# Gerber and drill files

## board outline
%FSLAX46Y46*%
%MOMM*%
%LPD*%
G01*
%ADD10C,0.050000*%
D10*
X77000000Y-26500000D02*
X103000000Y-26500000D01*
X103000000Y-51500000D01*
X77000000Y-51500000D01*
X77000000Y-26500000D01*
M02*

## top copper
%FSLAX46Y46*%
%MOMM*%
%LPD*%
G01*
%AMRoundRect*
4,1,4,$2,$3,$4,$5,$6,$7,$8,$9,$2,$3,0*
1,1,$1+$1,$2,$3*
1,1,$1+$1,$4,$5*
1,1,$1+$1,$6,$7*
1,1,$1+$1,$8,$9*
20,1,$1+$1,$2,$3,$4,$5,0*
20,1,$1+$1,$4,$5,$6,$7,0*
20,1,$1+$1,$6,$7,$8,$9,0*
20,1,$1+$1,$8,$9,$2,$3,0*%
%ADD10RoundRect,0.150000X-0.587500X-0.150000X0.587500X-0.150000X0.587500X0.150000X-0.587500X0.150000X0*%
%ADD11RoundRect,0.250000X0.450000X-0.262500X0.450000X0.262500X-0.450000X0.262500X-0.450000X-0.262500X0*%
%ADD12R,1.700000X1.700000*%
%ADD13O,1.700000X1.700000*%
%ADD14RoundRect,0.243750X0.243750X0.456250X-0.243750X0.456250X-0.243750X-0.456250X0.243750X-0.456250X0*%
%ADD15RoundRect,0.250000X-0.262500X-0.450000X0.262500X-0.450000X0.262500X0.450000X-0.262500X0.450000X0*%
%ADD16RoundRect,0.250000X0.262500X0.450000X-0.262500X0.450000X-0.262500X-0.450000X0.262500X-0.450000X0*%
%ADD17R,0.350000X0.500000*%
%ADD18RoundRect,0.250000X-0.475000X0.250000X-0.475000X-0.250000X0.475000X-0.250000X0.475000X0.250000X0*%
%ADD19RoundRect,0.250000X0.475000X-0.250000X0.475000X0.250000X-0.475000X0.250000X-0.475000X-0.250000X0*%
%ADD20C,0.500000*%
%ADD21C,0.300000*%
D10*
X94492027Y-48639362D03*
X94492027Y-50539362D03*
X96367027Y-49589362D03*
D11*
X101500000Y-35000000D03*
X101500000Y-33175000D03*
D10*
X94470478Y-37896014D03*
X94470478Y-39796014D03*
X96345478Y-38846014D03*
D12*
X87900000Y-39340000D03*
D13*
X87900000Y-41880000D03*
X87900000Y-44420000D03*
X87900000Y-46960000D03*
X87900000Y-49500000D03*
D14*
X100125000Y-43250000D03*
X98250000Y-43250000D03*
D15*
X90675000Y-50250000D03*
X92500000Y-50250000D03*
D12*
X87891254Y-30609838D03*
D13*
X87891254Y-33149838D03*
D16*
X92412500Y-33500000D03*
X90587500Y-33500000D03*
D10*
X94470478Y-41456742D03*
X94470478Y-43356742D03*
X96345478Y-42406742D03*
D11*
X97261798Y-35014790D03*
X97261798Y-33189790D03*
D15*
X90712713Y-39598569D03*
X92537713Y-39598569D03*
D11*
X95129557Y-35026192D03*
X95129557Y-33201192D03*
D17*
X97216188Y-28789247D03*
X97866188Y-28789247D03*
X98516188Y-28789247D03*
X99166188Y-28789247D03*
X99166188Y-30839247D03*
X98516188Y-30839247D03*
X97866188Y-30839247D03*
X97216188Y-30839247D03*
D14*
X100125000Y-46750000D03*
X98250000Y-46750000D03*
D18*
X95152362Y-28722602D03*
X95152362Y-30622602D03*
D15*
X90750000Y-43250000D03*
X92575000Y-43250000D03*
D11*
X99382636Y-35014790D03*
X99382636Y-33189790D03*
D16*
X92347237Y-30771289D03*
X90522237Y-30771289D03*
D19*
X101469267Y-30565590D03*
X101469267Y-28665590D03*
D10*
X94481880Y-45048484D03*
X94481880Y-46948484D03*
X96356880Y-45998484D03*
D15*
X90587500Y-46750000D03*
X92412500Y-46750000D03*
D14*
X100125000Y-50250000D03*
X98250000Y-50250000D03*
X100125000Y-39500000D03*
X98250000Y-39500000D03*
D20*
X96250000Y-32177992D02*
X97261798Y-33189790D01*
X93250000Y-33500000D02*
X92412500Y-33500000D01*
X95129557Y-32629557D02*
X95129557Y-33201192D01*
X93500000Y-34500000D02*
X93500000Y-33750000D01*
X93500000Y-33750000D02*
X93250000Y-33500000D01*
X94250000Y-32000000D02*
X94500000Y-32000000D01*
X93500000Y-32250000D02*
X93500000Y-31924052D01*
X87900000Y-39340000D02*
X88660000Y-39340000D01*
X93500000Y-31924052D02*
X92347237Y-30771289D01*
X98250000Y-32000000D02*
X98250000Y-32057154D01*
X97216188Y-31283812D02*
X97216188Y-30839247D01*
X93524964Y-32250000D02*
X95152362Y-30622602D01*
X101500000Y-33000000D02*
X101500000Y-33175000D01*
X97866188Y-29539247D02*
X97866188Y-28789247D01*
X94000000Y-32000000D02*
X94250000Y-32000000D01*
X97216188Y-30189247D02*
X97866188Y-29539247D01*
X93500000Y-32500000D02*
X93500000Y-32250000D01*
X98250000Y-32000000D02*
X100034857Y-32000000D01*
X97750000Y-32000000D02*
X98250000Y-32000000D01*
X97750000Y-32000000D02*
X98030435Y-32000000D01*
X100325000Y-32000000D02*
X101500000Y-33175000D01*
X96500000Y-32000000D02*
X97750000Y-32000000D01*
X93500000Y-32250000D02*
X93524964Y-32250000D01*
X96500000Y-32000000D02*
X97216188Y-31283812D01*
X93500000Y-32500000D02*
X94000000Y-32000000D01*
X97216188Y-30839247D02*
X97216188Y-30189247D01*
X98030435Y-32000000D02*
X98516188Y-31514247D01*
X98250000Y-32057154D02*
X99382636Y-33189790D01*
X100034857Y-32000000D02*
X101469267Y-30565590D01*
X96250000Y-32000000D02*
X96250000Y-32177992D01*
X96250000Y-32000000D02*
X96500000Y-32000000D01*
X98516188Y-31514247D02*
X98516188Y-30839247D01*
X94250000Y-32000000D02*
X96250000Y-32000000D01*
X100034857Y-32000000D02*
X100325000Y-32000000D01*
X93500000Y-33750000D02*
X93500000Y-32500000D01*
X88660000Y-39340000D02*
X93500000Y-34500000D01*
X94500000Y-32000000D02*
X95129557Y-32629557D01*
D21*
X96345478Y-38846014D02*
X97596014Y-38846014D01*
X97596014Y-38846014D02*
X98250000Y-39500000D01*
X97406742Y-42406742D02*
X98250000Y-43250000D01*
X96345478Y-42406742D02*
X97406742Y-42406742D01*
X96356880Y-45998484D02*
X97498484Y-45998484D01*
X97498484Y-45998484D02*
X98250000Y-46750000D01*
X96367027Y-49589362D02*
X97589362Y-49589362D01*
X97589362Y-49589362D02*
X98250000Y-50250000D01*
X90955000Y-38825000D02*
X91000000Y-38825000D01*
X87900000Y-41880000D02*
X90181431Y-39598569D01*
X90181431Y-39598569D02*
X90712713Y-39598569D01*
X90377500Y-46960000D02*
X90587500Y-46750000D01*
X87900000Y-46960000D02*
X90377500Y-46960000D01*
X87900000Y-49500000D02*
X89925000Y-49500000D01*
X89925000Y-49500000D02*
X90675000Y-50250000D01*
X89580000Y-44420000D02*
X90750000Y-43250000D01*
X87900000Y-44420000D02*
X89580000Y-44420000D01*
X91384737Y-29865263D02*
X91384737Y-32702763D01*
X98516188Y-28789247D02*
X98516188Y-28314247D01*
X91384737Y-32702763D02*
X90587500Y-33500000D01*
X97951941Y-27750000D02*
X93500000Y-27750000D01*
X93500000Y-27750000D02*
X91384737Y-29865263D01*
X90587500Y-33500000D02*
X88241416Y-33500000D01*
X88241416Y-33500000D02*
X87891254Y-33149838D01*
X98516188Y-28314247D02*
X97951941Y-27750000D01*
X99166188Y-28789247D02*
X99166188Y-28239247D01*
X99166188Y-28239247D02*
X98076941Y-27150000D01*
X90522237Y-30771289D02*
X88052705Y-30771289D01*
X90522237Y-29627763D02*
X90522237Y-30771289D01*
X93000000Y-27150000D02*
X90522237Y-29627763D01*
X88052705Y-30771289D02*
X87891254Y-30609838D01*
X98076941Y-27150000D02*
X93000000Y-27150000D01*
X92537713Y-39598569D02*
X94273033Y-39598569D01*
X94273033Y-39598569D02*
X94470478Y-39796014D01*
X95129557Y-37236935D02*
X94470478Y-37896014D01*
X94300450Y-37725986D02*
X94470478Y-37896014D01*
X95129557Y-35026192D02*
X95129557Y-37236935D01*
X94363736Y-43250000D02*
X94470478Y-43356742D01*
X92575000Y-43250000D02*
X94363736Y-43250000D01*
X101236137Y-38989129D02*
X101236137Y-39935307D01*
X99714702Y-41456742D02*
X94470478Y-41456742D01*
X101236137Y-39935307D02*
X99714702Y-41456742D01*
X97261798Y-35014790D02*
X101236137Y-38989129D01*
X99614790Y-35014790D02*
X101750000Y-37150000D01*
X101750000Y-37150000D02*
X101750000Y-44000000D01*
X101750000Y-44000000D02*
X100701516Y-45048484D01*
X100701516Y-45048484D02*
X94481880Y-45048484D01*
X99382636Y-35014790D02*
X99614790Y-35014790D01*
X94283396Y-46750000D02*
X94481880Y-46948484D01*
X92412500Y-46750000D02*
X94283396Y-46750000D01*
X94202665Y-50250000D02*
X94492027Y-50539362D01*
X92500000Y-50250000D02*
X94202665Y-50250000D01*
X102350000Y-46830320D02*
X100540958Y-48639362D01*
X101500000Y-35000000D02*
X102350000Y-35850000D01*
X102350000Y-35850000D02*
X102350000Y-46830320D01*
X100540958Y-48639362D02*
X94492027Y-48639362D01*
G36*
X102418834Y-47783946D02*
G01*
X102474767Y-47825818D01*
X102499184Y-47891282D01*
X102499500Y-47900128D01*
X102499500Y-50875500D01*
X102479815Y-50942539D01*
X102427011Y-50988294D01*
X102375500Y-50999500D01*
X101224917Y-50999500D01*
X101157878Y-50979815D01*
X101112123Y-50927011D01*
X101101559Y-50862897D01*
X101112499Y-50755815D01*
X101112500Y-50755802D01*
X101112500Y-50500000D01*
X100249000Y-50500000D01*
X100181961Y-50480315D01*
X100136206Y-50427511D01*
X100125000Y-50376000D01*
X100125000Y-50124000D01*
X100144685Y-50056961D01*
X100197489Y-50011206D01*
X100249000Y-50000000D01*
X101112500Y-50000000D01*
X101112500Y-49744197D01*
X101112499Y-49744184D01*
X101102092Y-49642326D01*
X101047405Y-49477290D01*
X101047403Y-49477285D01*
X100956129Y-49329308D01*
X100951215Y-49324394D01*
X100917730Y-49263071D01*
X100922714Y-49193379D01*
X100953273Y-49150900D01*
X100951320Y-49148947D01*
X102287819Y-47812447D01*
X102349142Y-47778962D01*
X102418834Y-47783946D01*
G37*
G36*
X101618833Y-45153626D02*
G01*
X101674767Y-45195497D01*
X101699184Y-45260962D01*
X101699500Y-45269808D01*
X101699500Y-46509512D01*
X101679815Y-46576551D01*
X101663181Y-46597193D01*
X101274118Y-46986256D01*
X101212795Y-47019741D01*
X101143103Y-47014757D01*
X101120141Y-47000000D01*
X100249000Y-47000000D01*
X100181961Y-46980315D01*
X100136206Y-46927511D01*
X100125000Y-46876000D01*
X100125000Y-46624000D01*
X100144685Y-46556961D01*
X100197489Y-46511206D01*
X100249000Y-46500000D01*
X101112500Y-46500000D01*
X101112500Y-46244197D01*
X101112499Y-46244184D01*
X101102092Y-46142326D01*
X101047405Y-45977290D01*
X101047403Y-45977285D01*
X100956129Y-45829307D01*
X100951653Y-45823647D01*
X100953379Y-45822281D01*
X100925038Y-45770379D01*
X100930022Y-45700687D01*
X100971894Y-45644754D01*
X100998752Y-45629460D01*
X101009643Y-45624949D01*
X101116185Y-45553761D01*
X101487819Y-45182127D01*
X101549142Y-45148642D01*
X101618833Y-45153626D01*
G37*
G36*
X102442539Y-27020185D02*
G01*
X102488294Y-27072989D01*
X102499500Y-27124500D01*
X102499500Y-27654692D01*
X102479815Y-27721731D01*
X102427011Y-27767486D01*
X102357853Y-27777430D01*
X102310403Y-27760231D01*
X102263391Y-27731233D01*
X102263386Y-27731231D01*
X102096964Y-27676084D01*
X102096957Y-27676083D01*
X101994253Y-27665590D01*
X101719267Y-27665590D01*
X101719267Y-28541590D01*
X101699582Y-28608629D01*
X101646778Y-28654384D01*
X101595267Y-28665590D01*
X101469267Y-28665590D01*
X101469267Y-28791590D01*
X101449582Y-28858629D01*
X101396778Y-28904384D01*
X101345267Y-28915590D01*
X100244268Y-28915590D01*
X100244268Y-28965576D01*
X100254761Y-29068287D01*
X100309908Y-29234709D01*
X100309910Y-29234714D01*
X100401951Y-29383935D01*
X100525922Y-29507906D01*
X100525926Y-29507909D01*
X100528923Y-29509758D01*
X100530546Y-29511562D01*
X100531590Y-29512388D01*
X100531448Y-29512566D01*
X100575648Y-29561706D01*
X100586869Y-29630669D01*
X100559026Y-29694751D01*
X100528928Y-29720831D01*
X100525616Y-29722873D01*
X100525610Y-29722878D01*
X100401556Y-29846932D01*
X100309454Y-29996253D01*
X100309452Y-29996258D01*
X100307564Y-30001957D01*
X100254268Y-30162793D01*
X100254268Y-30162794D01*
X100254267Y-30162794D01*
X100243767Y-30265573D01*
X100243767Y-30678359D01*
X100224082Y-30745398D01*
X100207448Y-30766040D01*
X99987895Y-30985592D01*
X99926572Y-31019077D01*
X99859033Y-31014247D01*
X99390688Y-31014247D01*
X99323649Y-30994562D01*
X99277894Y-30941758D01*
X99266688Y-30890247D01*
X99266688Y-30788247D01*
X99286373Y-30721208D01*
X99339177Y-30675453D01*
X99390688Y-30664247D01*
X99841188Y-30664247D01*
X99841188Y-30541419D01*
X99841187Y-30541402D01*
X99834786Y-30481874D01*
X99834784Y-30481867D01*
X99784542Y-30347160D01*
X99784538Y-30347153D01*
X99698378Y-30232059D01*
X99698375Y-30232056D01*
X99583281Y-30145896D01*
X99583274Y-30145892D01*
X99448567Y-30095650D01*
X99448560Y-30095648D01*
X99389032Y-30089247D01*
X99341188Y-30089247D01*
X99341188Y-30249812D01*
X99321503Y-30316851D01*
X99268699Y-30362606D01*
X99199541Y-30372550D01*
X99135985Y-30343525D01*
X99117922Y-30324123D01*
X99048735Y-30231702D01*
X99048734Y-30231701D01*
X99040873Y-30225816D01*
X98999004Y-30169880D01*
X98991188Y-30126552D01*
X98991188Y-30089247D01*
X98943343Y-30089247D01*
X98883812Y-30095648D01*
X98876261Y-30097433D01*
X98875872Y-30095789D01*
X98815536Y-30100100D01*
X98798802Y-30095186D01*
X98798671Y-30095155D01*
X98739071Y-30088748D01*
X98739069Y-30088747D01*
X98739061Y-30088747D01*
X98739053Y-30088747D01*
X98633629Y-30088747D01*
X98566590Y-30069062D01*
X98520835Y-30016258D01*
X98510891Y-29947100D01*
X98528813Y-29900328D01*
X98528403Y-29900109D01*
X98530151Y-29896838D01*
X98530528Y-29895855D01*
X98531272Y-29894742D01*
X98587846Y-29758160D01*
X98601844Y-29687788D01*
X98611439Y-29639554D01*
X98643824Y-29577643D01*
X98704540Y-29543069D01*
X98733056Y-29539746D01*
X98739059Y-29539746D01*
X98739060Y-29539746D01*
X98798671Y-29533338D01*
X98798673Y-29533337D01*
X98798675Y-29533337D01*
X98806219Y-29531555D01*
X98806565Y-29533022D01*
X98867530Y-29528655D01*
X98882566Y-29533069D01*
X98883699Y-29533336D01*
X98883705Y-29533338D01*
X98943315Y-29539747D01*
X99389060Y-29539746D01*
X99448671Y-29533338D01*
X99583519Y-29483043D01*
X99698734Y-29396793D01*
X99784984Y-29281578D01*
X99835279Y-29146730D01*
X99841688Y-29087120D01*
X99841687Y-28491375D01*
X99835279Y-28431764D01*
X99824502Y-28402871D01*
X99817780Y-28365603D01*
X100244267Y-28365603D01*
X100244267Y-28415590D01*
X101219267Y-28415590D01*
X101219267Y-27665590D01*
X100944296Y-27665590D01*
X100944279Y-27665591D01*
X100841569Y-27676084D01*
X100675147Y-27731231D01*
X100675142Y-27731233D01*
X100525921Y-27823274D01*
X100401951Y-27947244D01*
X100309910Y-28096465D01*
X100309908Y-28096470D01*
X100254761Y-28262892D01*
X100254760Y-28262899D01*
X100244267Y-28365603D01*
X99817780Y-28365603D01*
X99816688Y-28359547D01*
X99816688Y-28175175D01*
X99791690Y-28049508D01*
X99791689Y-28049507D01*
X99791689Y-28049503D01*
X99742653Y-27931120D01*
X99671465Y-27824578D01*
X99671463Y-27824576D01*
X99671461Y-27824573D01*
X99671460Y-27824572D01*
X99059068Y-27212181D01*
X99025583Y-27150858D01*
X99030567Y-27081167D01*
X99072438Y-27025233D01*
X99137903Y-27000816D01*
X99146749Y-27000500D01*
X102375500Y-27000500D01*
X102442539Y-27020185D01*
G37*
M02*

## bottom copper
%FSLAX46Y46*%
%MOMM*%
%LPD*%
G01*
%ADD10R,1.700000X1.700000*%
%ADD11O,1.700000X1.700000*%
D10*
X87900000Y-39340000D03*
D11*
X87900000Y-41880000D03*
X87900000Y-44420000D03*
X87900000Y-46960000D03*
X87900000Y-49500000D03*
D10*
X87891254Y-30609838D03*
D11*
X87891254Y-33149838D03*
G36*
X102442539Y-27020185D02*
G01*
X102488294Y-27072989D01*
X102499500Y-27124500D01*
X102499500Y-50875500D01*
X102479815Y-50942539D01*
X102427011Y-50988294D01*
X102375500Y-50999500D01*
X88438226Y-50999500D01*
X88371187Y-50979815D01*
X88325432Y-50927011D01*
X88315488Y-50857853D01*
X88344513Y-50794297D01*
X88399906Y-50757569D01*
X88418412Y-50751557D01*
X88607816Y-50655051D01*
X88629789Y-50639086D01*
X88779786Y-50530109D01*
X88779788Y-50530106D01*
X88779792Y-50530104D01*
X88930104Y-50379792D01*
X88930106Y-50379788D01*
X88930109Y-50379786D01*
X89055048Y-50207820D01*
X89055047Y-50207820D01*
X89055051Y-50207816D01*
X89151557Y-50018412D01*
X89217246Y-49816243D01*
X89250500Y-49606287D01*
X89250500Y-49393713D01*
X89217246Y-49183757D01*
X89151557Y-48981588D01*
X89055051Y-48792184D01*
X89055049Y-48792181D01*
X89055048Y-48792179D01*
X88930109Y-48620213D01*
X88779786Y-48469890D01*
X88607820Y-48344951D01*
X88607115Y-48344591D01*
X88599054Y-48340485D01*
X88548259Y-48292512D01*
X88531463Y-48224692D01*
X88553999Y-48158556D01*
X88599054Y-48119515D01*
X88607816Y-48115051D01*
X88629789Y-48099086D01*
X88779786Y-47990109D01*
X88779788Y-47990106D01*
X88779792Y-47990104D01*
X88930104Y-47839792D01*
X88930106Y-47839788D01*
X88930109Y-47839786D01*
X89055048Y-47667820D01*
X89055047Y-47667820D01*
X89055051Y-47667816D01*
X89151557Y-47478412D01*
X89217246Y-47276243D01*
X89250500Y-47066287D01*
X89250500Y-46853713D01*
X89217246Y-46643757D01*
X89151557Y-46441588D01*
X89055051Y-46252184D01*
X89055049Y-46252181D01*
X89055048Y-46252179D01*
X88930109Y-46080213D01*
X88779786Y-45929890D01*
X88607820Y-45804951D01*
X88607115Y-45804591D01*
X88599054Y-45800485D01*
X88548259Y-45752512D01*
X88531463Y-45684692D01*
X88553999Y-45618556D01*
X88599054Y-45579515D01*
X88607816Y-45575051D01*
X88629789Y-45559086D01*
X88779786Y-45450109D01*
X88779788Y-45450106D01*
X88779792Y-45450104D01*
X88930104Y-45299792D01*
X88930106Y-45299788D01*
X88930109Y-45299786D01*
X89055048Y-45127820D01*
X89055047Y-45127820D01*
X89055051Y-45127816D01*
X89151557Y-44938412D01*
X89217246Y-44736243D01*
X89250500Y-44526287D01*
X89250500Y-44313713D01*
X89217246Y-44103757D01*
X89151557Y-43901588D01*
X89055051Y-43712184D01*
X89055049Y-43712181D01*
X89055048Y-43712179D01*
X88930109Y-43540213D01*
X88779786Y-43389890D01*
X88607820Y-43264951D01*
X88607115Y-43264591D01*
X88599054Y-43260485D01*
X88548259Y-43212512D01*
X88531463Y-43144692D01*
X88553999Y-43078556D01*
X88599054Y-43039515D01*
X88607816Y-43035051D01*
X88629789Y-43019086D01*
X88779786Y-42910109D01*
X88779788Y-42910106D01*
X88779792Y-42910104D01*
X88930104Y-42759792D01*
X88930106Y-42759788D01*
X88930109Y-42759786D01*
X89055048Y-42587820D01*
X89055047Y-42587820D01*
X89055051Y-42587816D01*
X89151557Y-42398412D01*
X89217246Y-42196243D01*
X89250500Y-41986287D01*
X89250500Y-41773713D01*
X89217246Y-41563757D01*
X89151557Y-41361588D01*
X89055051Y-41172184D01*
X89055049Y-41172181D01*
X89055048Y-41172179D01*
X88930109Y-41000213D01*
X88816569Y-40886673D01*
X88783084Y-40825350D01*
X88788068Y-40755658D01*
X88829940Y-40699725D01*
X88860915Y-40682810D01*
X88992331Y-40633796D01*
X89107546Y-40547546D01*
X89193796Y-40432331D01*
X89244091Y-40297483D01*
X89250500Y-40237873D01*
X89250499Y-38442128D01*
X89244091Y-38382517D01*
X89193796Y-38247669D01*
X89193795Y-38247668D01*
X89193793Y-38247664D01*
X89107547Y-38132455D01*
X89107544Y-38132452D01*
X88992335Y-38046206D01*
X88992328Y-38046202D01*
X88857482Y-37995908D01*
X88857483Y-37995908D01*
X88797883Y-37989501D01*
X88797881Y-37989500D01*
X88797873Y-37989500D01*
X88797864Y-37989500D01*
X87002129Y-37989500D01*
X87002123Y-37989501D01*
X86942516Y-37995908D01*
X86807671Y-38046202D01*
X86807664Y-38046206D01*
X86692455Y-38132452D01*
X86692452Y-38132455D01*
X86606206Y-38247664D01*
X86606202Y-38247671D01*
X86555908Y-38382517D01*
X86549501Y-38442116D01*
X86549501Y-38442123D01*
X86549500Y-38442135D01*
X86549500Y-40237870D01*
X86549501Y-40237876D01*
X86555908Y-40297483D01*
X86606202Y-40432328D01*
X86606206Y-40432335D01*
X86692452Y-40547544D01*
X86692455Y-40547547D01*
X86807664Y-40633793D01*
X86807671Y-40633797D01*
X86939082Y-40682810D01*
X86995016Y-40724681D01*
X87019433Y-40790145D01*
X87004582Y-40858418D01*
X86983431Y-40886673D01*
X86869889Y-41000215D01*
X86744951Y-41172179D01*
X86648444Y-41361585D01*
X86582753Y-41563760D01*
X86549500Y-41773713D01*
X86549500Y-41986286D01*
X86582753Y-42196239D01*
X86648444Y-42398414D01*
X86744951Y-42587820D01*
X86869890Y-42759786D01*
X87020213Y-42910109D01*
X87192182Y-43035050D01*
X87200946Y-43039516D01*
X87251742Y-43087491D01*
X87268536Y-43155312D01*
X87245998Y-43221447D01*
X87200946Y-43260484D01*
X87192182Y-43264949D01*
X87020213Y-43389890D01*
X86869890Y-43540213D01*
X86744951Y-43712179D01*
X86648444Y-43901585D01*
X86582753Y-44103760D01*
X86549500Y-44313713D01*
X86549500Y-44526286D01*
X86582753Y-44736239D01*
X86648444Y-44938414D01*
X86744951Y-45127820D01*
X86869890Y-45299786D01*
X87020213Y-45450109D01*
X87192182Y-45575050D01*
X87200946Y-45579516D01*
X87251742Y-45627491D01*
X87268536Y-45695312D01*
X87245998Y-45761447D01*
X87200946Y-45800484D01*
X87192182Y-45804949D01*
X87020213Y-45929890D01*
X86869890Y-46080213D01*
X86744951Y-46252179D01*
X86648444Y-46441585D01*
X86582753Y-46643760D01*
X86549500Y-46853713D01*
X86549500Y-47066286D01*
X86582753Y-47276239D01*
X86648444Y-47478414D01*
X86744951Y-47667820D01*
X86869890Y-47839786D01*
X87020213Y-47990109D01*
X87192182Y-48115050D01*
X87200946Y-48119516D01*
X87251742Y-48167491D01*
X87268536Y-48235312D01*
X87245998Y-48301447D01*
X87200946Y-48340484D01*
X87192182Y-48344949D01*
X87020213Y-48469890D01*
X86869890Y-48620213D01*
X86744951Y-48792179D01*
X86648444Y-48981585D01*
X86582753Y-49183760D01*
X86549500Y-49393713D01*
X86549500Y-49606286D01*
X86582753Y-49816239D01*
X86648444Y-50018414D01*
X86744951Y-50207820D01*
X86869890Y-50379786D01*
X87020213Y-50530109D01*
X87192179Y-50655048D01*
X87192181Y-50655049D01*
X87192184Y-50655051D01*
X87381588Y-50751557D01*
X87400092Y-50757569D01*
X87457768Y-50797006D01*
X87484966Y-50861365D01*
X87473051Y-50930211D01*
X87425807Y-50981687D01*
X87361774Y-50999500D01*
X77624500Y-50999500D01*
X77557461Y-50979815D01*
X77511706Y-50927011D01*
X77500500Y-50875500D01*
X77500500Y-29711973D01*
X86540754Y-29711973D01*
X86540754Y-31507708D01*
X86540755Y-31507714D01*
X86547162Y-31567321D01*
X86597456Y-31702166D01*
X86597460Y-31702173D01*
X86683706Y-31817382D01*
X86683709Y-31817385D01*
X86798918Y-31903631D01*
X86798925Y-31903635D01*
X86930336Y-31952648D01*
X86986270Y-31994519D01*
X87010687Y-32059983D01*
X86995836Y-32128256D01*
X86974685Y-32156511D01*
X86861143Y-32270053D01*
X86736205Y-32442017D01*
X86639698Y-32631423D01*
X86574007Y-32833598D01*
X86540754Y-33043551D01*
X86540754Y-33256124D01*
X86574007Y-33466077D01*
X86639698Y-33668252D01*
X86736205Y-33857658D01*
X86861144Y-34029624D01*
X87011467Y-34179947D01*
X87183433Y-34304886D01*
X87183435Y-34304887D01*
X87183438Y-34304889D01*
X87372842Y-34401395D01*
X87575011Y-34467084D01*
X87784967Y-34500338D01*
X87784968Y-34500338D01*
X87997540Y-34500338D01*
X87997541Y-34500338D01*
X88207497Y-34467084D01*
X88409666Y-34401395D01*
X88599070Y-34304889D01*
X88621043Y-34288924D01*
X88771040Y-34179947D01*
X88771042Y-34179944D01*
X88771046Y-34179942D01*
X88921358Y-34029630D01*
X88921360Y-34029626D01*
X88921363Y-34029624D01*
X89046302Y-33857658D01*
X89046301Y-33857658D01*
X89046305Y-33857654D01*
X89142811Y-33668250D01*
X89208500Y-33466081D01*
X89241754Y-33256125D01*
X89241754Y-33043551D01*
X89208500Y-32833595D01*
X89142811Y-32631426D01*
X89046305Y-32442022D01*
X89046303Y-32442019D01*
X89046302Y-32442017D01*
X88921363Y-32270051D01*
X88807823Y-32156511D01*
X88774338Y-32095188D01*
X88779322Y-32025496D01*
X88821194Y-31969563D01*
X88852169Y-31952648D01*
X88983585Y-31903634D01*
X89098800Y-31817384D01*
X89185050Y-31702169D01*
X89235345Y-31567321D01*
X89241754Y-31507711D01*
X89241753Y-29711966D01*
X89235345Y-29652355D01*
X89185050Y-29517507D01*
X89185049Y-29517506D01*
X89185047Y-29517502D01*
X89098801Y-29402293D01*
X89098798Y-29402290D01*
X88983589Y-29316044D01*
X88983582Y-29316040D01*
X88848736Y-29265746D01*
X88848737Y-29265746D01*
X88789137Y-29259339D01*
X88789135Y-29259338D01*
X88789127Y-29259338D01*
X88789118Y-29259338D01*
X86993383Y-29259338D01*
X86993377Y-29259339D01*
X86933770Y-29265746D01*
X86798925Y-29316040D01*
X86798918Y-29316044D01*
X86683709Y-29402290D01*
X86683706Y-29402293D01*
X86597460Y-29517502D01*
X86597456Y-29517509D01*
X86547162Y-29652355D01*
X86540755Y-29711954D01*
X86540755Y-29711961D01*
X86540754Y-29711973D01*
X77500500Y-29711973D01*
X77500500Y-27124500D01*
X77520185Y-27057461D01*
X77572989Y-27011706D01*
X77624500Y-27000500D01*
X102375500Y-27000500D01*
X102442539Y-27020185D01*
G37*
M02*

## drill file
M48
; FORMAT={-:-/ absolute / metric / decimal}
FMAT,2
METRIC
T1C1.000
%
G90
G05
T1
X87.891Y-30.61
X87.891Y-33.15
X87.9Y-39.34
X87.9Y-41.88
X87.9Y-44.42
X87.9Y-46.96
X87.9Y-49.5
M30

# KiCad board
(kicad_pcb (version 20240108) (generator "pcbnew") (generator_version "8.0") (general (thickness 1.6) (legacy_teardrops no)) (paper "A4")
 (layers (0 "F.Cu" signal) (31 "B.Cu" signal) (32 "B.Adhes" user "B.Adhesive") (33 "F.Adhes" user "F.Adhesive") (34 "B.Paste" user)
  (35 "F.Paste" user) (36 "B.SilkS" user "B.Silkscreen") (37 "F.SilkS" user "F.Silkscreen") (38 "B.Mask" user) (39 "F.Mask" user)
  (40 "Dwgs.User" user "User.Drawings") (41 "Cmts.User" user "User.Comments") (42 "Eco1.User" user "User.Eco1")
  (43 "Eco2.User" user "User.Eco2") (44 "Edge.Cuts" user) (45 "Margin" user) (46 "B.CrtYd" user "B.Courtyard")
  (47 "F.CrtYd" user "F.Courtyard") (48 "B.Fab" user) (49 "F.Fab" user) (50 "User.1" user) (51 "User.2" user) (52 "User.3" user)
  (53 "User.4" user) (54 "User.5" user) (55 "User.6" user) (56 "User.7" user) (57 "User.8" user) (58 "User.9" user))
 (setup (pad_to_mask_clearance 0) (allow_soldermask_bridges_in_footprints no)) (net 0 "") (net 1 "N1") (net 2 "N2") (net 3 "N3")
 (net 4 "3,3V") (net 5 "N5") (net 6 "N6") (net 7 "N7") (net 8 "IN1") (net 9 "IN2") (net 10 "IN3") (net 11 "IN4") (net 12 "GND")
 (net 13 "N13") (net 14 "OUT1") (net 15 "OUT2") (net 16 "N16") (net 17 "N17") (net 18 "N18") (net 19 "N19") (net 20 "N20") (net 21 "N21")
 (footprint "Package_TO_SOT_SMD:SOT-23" (layer "F.Cu") (at 95.429527 49.589362)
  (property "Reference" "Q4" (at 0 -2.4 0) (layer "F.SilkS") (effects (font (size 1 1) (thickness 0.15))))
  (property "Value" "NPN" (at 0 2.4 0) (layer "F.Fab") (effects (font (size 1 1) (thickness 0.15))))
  (pad "1" smd roundrect (at -0.9375 -0.95) (size 1.475 0.6) (layers "F.Cu" "F.Paste" "F.Mask") (roundrect_rratio 0.25) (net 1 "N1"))
  (pad "2" smd roundrect (at -0.9375 0.95) (size 1.475 0.6) (layers "F.Cu" "F.Paste" "F.Mask") (roundrect_rratio 0.25) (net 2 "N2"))
  (pad "3" smd roundrect (at 0.9375 0) (size 1.475 0.6) (layers "F.Cu" "F.Paste" "F.Mask") (roundrect_rratio 0.25) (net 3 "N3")))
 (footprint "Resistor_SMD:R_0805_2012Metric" (layer "F.Cu") (at 101.5 34.0875 90)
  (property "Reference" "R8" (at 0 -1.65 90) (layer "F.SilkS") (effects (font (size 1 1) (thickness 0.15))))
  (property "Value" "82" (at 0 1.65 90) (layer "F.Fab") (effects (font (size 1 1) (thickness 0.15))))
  (pad "1" smd roundrect (at -0.9125 0 90) (size 1.025 1.4) (layers "F.Cu" "F.Paste" "F.Mask") (roundrect_rratio 0.243902) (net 1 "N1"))
  (pad "2" smd roundrect (at 0.9125 0 90) (size 1.025 1.4) (layers "F.Cu" "F.Paste" "F.Mask") (roundrect_rratio 0.243902) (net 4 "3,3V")))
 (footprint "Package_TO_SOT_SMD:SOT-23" (layer "F.Cu") (at 95.407978 38.846014)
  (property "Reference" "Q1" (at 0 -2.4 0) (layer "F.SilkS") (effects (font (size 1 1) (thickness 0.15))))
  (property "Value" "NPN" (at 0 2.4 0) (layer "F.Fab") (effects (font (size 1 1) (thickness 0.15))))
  (pad "1" smd roundrect (at -0.9375 -0.95) (size 1.475 0.6) (layers "F.Cu" "F.Paste" "F.Mask") (roundrect_rratio 0.25) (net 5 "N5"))
  (pad "2" smd roundrect (at -0.9375 0.95) (size 1.475 0.6) (layers "F.Cu" "F.Paste" "F.Mask") (roundrect_rratio 0.25) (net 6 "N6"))
  (pad "3" smd roundrect (at 0.9375 0) (size 1.475 0.6) (layers "F.Cu" "F.Paste" "F.Mask") (roundrect_rratio 0.25) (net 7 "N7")))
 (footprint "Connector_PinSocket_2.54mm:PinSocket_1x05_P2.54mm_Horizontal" (layer "F.Cu") (at 87.9 39.34)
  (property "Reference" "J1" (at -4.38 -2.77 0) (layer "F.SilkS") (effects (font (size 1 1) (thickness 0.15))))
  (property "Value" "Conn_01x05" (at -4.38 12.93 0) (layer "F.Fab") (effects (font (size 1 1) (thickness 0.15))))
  (pad "1" thru_hole rect (at 0 0) (size 1.7 1.7) (drill 1) (layers "*.Cu" "*.Mask") (remove_unused_layers no) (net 4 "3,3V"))
  (pad "2" thru_hole oval (at 0 2.54) (size 1.7 1.7) (drill 1) (layers "*.Cu" "*.Mask") (remove_unused_layers no) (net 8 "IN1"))
  (pad "3" thru_hole oval (at 0 5.08) (size 1.7 1.7) (drill 1) (layers "*.Cu" "*.Mask") (remove_unused_layers no) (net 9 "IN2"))
  (pad "4" thru_hole oval (at 0 7.62) (size 1.7 1.7) (drill 1) (layers "*.Cu" "*.Mask") (remove_unused_layers no) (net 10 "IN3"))
  (pad "5" thru_hole oval (at 0 10.16) (size 1.7 1.7) (drill 1) (layers "*.Cu" "*.Mask") (remove_unused_layers no) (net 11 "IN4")))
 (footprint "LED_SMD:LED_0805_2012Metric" (layer "F.Cu") (at 99.1875 43.25 180)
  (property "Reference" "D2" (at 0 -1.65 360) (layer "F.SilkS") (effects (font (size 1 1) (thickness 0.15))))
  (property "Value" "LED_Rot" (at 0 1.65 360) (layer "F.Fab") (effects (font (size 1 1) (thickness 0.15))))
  (pad "1" smd roundrect (at -0.9375 0 180) (size 0.975 1.4) (layers "F.Cu" "F.Paste" "F.Mask") (roundrect_rratio 0.25) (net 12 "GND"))
  (pad "2" smd roundrect (at 0.9375 0 180) (size 0.975 1.4) (layers "F.Cu" "F.Paste" "F.Mask") (roundrect_rratio 0.25) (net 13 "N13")))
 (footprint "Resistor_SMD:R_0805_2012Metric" (layer "F.Cu") (at 91.5875 50.25)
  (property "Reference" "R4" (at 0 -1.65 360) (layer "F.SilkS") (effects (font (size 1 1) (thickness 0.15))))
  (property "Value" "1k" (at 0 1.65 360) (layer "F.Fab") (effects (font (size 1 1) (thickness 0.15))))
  (pad "1" smd roundrect (at -0.9125 0) (size 1.025 1.4) (layers "F.Cu" "F.Paste" "F.Mask") (roundrect_rratio 0.243902) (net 11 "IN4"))
  (pad "2" smd roundrect (at 0.9125 0) (size 1.025 1.4) (layers "F.Cu" "F.Paste" "F.Mask") (roundrect_rratio 0.243902) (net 2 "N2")))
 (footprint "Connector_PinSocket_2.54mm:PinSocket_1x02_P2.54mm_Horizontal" (layer "F.Cu") (at 87.891254 30.609838)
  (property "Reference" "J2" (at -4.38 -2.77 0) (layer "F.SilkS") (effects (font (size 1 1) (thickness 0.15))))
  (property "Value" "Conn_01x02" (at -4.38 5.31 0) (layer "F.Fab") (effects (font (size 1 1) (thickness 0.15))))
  (pad "1" thru_hole rect (at 0 0) (size 1.7 1.7) (drill 1) (layers "*.Cu" "*.Mask") (remove_unused_layers no) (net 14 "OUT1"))
  (pad "2" thru_hole oval (at 0 2.54) (size 1.7 1.7) (drill 1) (layers "*.Cu" "*.Mask") (remove_unused_layers no) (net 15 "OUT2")))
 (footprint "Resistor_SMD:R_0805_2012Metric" (layer "F.Cu") (at 91.5 33.5 180)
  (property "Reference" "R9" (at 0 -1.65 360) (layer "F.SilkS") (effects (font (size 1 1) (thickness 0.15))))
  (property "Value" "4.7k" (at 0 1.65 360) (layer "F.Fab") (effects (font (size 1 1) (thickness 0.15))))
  (pad "1" smd roundrect (at -0.9125 0 180) (size 1.025 1.4) (layers "F.Cu" "F.Paste" "F.Mask") (roundrect_rratio 0.243902) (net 4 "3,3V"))
  (pad "2" smd roundrect (at 0.9125 0 180) (size 1.025 1.4) (layers "F.Cu" "F.Paste" "F.Mask") (roundrect_rratio 0.243902) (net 15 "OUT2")))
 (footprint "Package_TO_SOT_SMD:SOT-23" (layer "F.Cu") (at 95.407978 42.406742)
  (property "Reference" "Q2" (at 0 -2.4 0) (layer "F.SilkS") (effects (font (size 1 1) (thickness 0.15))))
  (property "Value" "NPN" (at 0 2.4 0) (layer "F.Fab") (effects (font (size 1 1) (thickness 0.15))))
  (pad "1" smd roundrect (at -0.9375 -0.95) (size 1.475 0.6) (layers "F.Cu" "F.Paste" "F.Mask") (roundrect_rratio 0.25) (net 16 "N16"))
  (pad "2" smd roundrect (at -0.9375 0.95) (size 1.475 0.6) (layers "F.Cu" "F.Paste" "F.Mask") (roundrect_rratio 0.25) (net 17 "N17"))
  (pad "3" smd roundrect (at 0.9375 0) (size 1.475 0.6) (layers "F.Cu" "F.Paste" "F.Mask") (roundrect_rratio 0.25) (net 13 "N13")))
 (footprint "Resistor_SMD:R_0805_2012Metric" (layer "F.Cu") (at 97.261798 34.10229 90)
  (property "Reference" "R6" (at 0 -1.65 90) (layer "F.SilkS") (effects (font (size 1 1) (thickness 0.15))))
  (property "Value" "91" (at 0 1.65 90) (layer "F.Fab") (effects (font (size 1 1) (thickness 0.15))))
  (pad "1" smd roundrect (at -0.9125 0 90) (size 1.025 1.4) (layers "F.Cu" "F.Paste" "F.Mask") (roundrect_rratio 0.243902) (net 16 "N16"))
  (pad "2" smd roundrect (at 0.9125 0 90) (size 1.025 1.4) (layers "F.Cu" "F.Paste" "F.Mask") (roundrect_rratio 0.243902) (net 4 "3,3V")))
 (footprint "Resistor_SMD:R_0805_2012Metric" (layer "F.Cu") (at 91.625213 39.598569)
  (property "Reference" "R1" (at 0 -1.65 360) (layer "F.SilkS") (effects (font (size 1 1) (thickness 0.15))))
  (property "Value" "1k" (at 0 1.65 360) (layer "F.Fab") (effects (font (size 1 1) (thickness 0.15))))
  (pad "1" smd roundrect (at -0.9125 0) (size 1.025 1.4) (layers "F.Cu" "F.Paste" "F.Mask") (roundrect_rratio 0.243902) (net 8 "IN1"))
  (pad "2" smd roundrect (at 0.9125 0) (size 1.025 1.4) (layers "F.Cu" "F.Paste" "F.Mask") (roundrect_rratio 0.243902) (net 6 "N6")))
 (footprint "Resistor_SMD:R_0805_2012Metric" (layer "F.Cu") (at 95.129557 34.113692 90)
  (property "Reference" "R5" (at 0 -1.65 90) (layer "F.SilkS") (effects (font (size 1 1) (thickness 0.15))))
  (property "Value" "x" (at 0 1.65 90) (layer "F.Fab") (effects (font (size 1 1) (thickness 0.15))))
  (pad "1" smd roundrect (at -0.9125 0 90) (size 1.025 1.4) (layers "F.Cu" "F.Paste" "F.Mask") (roundrect_rratio 0.243902) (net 5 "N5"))
  (pad "2" smd roundrect (at 0.9125 0 90) (size 1.025 1.4) (layers "F.Cu" "F.Paste" "F.Mask") (roundrect_rratio 0.243902) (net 4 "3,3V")))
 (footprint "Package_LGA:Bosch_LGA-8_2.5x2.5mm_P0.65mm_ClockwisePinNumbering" (layer "F.Cu") (at 98.191188 29.814247)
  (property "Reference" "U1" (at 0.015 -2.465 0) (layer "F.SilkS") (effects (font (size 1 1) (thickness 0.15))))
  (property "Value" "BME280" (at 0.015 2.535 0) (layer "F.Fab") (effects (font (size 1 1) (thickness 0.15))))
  (pad "1" smd rect (at -0.975 -1.025 90) (size 0.5 0.35) (layers "F.Cu" "F.Paste" "F.Mask") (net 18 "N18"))
  (pad "2" smd rect (at -0.325 -1.025 90) (size 0.5 0.35) (layers "F.Cu" "F.Paste" "F.Mask") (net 4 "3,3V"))
  (pad "3" smd rect (at 0.325 -1.025 90) (size 0.5 0.35) (layers "F.Cu" "F.Paste" "F.Mask") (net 15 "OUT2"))
  (pad "4" smd rect (at 0.975 -1.025 90) (size 0.5 0.35) (layers "F.Cu" "F.Paste" "F.Mask") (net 14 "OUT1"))
  (pad "5" smd rect (at 0.975 1.025 90) (size 0.5 0.35) (layers "F.Cu" "F.Paste" "F.Mask") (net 12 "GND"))
  (pad "6" smd rect (at 0.325 1.025 90) (size 0.5 0.35) (layers "F.Cu" "F.Paste" "F.Mask") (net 4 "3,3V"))
  (pad "7" smd rect (at -0.325 1.025 90) (size 0.5 0.35) (layers "F.Cu" "F.Paste" "F.Mask") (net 12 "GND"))
  (pad "8" smd rect (at -0.975 1.025 90) (size 0.5 0.35) (layers "F.Cu" "F.Paste" "F.Mask") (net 4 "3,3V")))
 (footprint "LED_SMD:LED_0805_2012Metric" (layer "F.Cu") (at 99.1875 46.75 180)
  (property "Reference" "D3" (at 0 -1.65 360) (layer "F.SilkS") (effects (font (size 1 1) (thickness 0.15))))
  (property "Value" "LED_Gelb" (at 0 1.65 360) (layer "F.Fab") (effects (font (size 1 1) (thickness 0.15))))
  (pad "1" smd roundrect (at -0.9375 0 180) (size 0.975 1.4) (layers "F.Cu" "F.Paste" "F.Mask") (roundrect_rratio 0.25) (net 12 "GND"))
  (pad "2" smd roundrect (at 0.9375 0 180) (size 0.975 1.4) (layers "F.Cu" "F.Paste" "F.Mask") (roundrect_rratio 0.25) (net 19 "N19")))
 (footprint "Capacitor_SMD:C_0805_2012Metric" (layer "F.Cu") (at 95.152362 29.672602 -90)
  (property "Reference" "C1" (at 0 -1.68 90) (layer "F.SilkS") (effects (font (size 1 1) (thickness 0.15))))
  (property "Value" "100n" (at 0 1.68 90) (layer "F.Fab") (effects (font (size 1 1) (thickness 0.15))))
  (pad "1" smd roundrect (at -0.95 0 270) (size 1 1.45) (layers "F.Cu" "F.Paste" "F.Mask") (roundrect_rratio 0.25) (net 18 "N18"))
  (pad "2" smd roundrect (at 0.95 0 270) (size 1 1.45) (layers "F.Cu" "F.Paste" "F.Mask") (roundrect_rratio 0.25) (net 4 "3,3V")))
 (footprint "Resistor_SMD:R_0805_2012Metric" (layer "F.Cu") (at 91.6625 43.25)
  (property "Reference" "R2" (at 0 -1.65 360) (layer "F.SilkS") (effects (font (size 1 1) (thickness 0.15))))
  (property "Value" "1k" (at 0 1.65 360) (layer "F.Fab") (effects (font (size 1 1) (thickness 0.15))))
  (pad "1" smd roundrect (at -0.9125 0) (size 1.025 1.4) (layers "F.Cu" "F.Paste" "F.Mask") (roundrect_rratio 0.243902) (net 9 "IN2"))
  (pad "2" smd roundrect (at 0.9125 0) (size 1.025 1.4) (layers "F.Cu" "F.Paste" "F.Mask") (roundrect_rratio 0.243902) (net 17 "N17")))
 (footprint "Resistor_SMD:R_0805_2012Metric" (layer "F.Cu") (at 99.382636 34.10229 90)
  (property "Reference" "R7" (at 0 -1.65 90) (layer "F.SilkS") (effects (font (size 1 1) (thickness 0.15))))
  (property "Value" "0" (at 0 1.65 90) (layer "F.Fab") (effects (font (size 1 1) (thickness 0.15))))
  (pad "1" smd roundrect (at -0.9125 0 90) (size 1.025 1.4) (layers "F.Cu" "F.Paste" "F.Mask") (roundrect_rratio 0.243902) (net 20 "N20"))
  (pad "2" smd roundrect (at 0.9125 0 90) (size 1.025 1.4) (layers "F.Cu" "F.Paste" "F.Mask") (roundrect_rratio 0.243902) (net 4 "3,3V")))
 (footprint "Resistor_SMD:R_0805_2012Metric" (layer "F.Cu") (at 91.434737 30.771289 180)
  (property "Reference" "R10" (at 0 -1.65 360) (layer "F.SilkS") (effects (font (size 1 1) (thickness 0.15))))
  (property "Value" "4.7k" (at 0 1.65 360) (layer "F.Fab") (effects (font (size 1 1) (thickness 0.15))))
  (pad "1" smd roundrect (at -0.9125 0 180) (size 1.025 1.4) (layers "F.Cu" "F.Paste" "F.Mask") (roundrect_rratio 0.243902) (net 4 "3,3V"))
  (pad "2" smd roundrect (at 0.9125 0 180) (size 1.025 1.4) (layers "F.Cu" "F.Paste" "F.Mask") (roundrect_rratio 0.243902) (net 14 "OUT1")))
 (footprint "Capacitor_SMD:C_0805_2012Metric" (layer "F.Cu") (at 101.469267 29.61559 90)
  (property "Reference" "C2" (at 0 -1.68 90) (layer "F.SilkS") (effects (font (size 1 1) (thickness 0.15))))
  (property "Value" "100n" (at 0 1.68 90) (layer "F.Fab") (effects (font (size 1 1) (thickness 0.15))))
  (pad "1" smd roundrect (at -0.95 0 90) (size 1 1.45) (layers "F.Cu" "F.Paste" "F.Mask") (roundrect_rratio 0.25) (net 4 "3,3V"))
  (pad "2" smd roundrect (at 0.95 0 90) (size 1 1.45) (layers "F.Cu" "F.Paste" "F.Mask") (roundrect_rratio 0.25) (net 12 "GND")))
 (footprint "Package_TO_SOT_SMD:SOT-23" (layer "F.Cu") (at 95.41938 45.998484)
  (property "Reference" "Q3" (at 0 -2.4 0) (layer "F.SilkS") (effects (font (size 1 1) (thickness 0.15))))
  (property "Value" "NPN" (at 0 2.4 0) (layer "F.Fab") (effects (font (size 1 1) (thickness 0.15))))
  (pad "1" smd roundrect (at -0.9375 -0.95) (size 1.475 0.6) (layers "F.Cu" "F.Paste" "F.Mask") (roundrect_rratio 0.25) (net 20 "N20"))
  (pad "2" smd roundrect (at -0.9375 0.95) (size 1.475 0.6) (layers "F.Cu" "F.Paste" "F.Mask") (roundrect_rratio 0.25) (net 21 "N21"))
  (pad "3" smd roundrect (at 0.9375 0) (size 1.475 0.6) (layers "F.Cu" "F.Paste" "F.Mask") (roundrect_rratio 0.25) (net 19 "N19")))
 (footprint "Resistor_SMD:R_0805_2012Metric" (layer "F.Cu") (at 91.5 46.75)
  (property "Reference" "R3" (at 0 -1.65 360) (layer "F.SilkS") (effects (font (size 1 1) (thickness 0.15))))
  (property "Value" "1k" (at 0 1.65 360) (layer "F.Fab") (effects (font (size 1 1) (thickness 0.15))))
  (pad "1" smd roundrect (at -0.9125 0) (size 1.025 1.4) (layers "F.Cu" "F.Paste" "F.Mask") (roundrect_rratio 0.243902) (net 10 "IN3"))
  (pad "2" smd roundrect (at 0.9125 0) (size 1.025 1.4) (layers "F.Cu" "F.Paste" "F.Mask") (roundrect_rratio 0.243902) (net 21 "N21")))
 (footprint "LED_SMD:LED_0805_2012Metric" (layer "F.Cu") (at 99.1875 50.25 180)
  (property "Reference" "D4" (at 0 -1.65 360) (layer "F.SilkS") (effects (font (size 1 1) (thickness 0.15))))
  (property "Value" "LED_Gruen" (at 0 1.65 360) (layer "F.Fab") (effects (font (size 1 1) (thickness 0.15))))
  (pad "1" smd roundrect (at -0.9375 0 180) (size 0.975 1.4) (layers "F.Cu" "F.Paste" "F.Mask") (roundrect_rratio 0.25) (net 12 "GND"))
  (pad "2" smd roundrect (at 0.9375 0 180) (size 0.975 1.4) (layers "F.Cu" "F.Paste" "F.Mask") (roundrect_rratio 0.25) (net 3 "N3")))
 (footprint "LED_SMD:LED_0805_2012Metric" (layer "F.Cu") (at 99.1875 39.5 180)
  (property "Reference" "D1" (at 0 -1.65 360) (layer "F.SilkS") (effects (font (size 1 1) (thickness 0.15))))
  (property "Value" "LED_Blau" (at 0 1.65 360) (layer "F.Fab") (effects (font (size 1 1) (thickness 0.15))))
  (pad "1" smd roundrect (at -0.9375 0 180) (size 0.975 1.4) (layers "F.Cu" "F.Paste" "F.Mask") (roundrect_rratio 0.25) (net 12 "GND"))
  (pad "2" smd roundrect (at 0.9375 0 180) (size 0.975 1.4) (layers "F.Cu" "F.Paste" "F.Mask") (roundrect_rratio 0.25) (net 7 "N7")))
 (gr_rect (start 77 26.5) (end 103 51.5) (stroke (width 0.05) (type default)) (fill none) (layer "Edge.Cuts"))
 (segment (start 96.25 32.177992) (end 97.261798 33.18979) (width 0.5) (layer "F.Cu") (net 4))
 (segment (start 93.25 33.5) (end 92.4125 33.5) (width 0.5) (layer "F.Cu") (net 4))
 (segment (start 95.129557 32.629557) (end 95.129557 33.201192) (width 0.5) (layer "F.Cu") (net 4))
 (segment (start 93.5 34.5) (end 93.5 33.75) (width 0.5) (layer "F.Cu") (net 4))
 (segment (start 93.5 33.75) (end 93.25 33.5) (width 0.5) (layer "F.Cu") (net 4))
 (segment (start 94.25 32) (end 94.5 32) (width 0.5) (layer "F.Cu") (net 4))
 (segment (start 93.5 32.25) (end 93.5 31.924052) (width 0.5) (layer "F.Cu") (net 4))
 (segment (start 87.9 39.34) (end 88.66 39.34) (width 0.5) (layer "F.Cu") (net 4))
 (segment (start 93.5 31.924052) (end 92.347237 30.771289) (width 0.5) (layer "F.Cu") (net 4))
 (segment (start 98.25 32) (end 98.25 32.057154) (width 0.5) (layer "F.Cu") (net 4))
 (segment (start 97.216188 31.283812) (end 97.216188 30.839247) (width 0.5) (layer "F.Cu") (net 4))
 (segment (start 93.524964 32.25) (end 95.152362 30.622602) (width 0.5) (layer "F.Cu") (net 4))
 (segment (start 101.5 33) (end 101.5 33.175) (width 0.5) (layer "F.Cu") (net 4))
 (segment (start 97.866188 29.539247) (end 97.866188 28.789247) (width 0.5) (layer "F.Cu") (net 4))
 (segment (start 94 32) (end 94.25 32) (width 0.5) (layer "F.Cu") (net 4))
 (segment (start 97.216188 30.189247) (end 97.866188 29.539247) (width 0.5) (layer "F.Cu") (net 4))
 (segment (start 93.5 32.5) (end 93.5 32.25) (width 0.5) (layer "F.Cu") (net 4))
 (segment (start 98.25 32) (end 100.034857 32) (width 0.5) (layer "F.Cu") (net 4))
 (segment (start 97.75 32) (end 98.25 32) (width 0.5) (layer "F.Cu") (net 4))
 (segment (start 97.75 32) (end 98.030435 32) (width 0.5) (layer "F.Cu") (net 4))
 (segment (start 100.325 32) (end 101.5 33.175) (width 0.5) (layer "F.Cu") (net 4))
 (segment (start 96.5 32) (end 97.75 32) (width 0.5) (layer "F.Cu") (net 4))
 (segment (start 93.5 32.25) (end 93.524964 32.25) (width 0.5) (layer "F.Cu") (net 4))
 (segment (start 96.5 32) (end 97.216188 31.283812) (width 0.5) (layer "F.Cu") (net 4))
 (segment (start 93.5 32.5) (end 94 32) (width 0.5) (layer "F.Cu") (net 4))
 (segment (start 97.216188 30.839247) (end 97.216188 30.189247) (width 0.5) (layer "F.Cu") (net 4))
 (segment (start 98.030435 32) (end 98.516188 31.514247) (width 0.5) (layer "F.Cu") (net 4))
 (segment (start 98.25 32.057154) (end 99.382636 33.18979) (width 0.5) (layer "F.Cu") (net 4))
 (segment (start 100.034857 32) (end 101.469267 30.56559) (width 0.5) (layer "F.Cu") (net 4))
 (segment (start 96.25 32) (end 96.25 32.177992) (width 0.5) (layer "F.Cu") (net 4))
 (segment (start 96.25 32) (end 96.5 32) (width 0.5) (layer "F.Cu") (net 4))
 (segment (start 98.516188 31.514247) (end 98.516188 30.839247) (width 0.5) (layer "F.Cu") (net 4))
 (segment (start 94.25 32) (end 96.25 32) (width 0.5) (layer "F.Cu") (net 4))
 (segment (start 100.034857 32) (end 100.325 32) (width 0.5) (layer "F.Cu") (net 4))
 (segment (start 93.5 33.75) (end 93.5 32.5) (width 0.5) (layer "F.Cu") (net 4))
 (segment (start 88.66 39.34) (end 93.5 34.5) (width 0.5) (layer "F.Cu") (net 4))
 (segment (start 94.5 32) (end 95.129557 32.629557) (width 0.5) (layer "F.Cu") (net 4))
 (segment (start 96.345478 38.846014) (end 97.596014 38.846014) (width 0.3) (layer "F.Cu") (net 7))
 (segment (start 97.596014 38.846014) (end 98.25 39.5) (width 0.3) (layer "F.Cu") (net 7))
 (segment (start 97.406742 42.406742) (end 98.25 43.25) (width 0.3) (layer "F.Cu") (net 13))
 (segment (start 96.345478 42.406742) (end 97.406742 42.406742) (width 0.3) (layer "F.Cu") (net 13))
 (segment (start 96.35688 45.998484) (end 97.498484 45.998484) (width 0.3) (layer "F.Cu") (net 19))
 (segment (start 97.498484 45.998484) (end 98.25 46.75) (width 0.3) (layer "F.Cu") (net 19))
 (segment (start 96.367027 49.589362) (end 97.589362 49.589362) (width 0.3) (layer "F.Cu") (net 3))
 (segment (start 97.589362 49.589362) (end 98.25 50.25) (width 0.3) (layer "F.Cu") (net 3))
 (segment (start 90.955 38.825) (end 91 38.825) (width 0.3) (layer "F.Cu") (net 8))
 (segment (start 87.9 41.88) (end 90.181431 39.598569) (width 0.3) (layer "F.Cu") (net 8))
 (segment (start 90.181431 39.598569) (end 90.712713 39.598569) (width 0.3) (layer "F.Cu") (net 8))
 (segment (start 90.3775 46.96) (end 90.5875 46.75) (width 0.3) (layer "F.Cu") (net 10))
 (segment (start 87.9 46.96) (end 90.3775 46.96) (width 0.3) (layer "F.Cu") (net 10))
 (segment (start 87.9 49.5) (end 89.925 49.5) (width 0.3) (layer "F.Cu") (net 11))
 (segment (start 89.925 49.5) (end 90.675 50.25) (width 0.3) (layer "F.Cu") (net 11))
 (segment (start 89.58 44.42) (end 90.75 43.25) (width 0.3) (layer "F.Cu") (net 9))
 (segment (start 87.9 44.42) (end 89.58 44.42) (width 0.3) (layer "F.Cu") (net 9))
 (segment (start 91.384737 29.865263) (end 91.384737 32.702763) (width 0.3) (layer "F.Cu") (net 15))
 (segment (start 98.516188 28.789247) (end 98.516188 28.314247) (width 0.3) (layer "F.Cu") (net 15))
 (segment (start 91.384737 32.702763) (end 90.5875 33.5) (width 0.3) (layer "F.Cu") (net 15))
 (segment (start 97.951941 27.75) (end 93.5 27.75) (width 0.3) (layer "F.Cu") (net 15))
 (segment (start 93.5 27.75) (end 91.384737 29.865263) (width 0.3) (layer "F.Cu") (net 15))
 (segment (start 90.5875 33.5) (end 88.241416 33.5) (width 0.3) (layer "F.Cu") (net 15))
 (segment (start 88.241416 33.5) (end 87.891254 33.149838) (width 0.3) (layer "F.Cu") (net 15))
 (segment (start 98.516188 28.314247) (end 97.951941 27.75) (width 0.3) (layer "F.Cu") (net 15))
 (segment (start 99.166188 28.789247) (end 99.166188 28.239247) (width 0.3) (layer "F.Cu") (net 14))
 (segment (start 99.166188 28.239247) (end 98.076941 27.15) (width 0.3) (layer "F.Cu") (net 14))
 (segment (start 90.522237 30.771289) (end 88.052705 30.771289) (width 0.3) (layer "F.Cu") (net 14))
 (segment (start 90.522237 29.627763) (end 90.522237 30.771289) (width 0.3) (layer "F.Cu") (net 14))
 (segment (start 93 27.15) (end 90.522237 29.627763) (width 0.3) (layer "F.Cu") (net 14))
 (segment (start 88.052705 30.771289) (end 87.891254 30.609838) (width 0.3) (layer "F.Cu") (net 14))
 (segment (start 98.076941 27.15) (end 93 27.15) (width 0.3) (layer "F.Cu") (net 14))
 (segment (start 92.537713 39.598569) (end 94.273033 39.598569) (width 0.3) (layer "F.Cu") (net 6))
 (segment (start 94.273033 39.598569) (end 94.470478 39.796014) (width 0.3) (layer "F.Cu") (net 6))
 (segment (start 95.129557 37.236935) (end 94.470478 37.896014) (width 0.3) (layer "F.Cu") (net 5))
 (segment (start 94.30045 37.725986) (end 94.470478 37.896014) (width 0.3) (layer "F.Cu") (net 5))
 (segment (start 95.129557 35.026192) (end 95.129557 37.236935) (width 0.3) (layer "F.Cu") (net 5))
 (segment (start 94.363736 43.25) (end 94.470478 43.356742) (width 0.3) (layer "F.Cu") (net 17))
 (segment (start 92.575 43.25) (end 94.363736 43.25) (width 0.3) (layer "F.Cu") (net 17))
 (segment (start 101.236137 38.989129) (end 101.236137 39.935307) (width 0.3) (layer "F.Cu") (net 16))
 (segment (start 99.714702 41.456742) (end 94.470478 41.456742) (width 0.3) (layer "F.Cu") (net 16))
 (segment (start 101.236137 39.935307) (end 99.714702 41.456742) (width 0.3) (layer "F.Cu") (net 16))
 (segment (start 97.261798 35.01479) (end 101.236137 38.989129) (width 0.3) (layer "F.Cu") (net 16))
 (segment (start 99.61479 35.01479) (end 101.75 37.15) (width 0.3) (layer "F.Cu") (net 20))
 (segment (start 101.75 37.15) (end 101.75 44) (width 0.3) (layer "F.Cu") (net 20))
 (segment (start 101.75 44) (end 100.701516 45.048484) (width 0.3) (layer "F.Cu") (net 20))
 (segment (start 100.701516 45.048484) (end 94.48188 45.048484) (width 0.3) (layer "F.Cu") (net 20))
 (segment (start 99.382636 35.01479) (end 99.61479 35.01479) (width 0.3) (layer "F.Cu") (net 20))
 (segment (start 94.283396 46.75) (end 94.48188 46.948484) (width 0.3) (layer "F.Cu") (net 21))
 (segment (start 92.4125 46.75) (end 94.283396 46.75) (width 0.3) (layer "F.Cu") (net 21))
 (segment (start 94.202665 50.25) (end 94.492027 50.539362) (width 0.3) (layer "F.Cu") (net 2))
 (segment (start 92.5 50.25) (end 94.202665 50.25) (width 0.3) (layer "F.Cu") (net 2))
 (segment (start 102.35 46.83032) (end 100.540958 48.639362) (width 0.3) (layer "F.Cu") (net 1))
 (segment (start 101.5 35) (end 102.35 35.85) (width 0.3) (layer "F.Cu") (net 1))
 (segment (start 102.35 35.85) (end 102.35 46.83032) (width 0.3) (layer "F.Cu") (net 1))
 (segment (start 100.540958 48.639362) (end 94.492027 48.639362) (width 0.3) (layer "F.Cu") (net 1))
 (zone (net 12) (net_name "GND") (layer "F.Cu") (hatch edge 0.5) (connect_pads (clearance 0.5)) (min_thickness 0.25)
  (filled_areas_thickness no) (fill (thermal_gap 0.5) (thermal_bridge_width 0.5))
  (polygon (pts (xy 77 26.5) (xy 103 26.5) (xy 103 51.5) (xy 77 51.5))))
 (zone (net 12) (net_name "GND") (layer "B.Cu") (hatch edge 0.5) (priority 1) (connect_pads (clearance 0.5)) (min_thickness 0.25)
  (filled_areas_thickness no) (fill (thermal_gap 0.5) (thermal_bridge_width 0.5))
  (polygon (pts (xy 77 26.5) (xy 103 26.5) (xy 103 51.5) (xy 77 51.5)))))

